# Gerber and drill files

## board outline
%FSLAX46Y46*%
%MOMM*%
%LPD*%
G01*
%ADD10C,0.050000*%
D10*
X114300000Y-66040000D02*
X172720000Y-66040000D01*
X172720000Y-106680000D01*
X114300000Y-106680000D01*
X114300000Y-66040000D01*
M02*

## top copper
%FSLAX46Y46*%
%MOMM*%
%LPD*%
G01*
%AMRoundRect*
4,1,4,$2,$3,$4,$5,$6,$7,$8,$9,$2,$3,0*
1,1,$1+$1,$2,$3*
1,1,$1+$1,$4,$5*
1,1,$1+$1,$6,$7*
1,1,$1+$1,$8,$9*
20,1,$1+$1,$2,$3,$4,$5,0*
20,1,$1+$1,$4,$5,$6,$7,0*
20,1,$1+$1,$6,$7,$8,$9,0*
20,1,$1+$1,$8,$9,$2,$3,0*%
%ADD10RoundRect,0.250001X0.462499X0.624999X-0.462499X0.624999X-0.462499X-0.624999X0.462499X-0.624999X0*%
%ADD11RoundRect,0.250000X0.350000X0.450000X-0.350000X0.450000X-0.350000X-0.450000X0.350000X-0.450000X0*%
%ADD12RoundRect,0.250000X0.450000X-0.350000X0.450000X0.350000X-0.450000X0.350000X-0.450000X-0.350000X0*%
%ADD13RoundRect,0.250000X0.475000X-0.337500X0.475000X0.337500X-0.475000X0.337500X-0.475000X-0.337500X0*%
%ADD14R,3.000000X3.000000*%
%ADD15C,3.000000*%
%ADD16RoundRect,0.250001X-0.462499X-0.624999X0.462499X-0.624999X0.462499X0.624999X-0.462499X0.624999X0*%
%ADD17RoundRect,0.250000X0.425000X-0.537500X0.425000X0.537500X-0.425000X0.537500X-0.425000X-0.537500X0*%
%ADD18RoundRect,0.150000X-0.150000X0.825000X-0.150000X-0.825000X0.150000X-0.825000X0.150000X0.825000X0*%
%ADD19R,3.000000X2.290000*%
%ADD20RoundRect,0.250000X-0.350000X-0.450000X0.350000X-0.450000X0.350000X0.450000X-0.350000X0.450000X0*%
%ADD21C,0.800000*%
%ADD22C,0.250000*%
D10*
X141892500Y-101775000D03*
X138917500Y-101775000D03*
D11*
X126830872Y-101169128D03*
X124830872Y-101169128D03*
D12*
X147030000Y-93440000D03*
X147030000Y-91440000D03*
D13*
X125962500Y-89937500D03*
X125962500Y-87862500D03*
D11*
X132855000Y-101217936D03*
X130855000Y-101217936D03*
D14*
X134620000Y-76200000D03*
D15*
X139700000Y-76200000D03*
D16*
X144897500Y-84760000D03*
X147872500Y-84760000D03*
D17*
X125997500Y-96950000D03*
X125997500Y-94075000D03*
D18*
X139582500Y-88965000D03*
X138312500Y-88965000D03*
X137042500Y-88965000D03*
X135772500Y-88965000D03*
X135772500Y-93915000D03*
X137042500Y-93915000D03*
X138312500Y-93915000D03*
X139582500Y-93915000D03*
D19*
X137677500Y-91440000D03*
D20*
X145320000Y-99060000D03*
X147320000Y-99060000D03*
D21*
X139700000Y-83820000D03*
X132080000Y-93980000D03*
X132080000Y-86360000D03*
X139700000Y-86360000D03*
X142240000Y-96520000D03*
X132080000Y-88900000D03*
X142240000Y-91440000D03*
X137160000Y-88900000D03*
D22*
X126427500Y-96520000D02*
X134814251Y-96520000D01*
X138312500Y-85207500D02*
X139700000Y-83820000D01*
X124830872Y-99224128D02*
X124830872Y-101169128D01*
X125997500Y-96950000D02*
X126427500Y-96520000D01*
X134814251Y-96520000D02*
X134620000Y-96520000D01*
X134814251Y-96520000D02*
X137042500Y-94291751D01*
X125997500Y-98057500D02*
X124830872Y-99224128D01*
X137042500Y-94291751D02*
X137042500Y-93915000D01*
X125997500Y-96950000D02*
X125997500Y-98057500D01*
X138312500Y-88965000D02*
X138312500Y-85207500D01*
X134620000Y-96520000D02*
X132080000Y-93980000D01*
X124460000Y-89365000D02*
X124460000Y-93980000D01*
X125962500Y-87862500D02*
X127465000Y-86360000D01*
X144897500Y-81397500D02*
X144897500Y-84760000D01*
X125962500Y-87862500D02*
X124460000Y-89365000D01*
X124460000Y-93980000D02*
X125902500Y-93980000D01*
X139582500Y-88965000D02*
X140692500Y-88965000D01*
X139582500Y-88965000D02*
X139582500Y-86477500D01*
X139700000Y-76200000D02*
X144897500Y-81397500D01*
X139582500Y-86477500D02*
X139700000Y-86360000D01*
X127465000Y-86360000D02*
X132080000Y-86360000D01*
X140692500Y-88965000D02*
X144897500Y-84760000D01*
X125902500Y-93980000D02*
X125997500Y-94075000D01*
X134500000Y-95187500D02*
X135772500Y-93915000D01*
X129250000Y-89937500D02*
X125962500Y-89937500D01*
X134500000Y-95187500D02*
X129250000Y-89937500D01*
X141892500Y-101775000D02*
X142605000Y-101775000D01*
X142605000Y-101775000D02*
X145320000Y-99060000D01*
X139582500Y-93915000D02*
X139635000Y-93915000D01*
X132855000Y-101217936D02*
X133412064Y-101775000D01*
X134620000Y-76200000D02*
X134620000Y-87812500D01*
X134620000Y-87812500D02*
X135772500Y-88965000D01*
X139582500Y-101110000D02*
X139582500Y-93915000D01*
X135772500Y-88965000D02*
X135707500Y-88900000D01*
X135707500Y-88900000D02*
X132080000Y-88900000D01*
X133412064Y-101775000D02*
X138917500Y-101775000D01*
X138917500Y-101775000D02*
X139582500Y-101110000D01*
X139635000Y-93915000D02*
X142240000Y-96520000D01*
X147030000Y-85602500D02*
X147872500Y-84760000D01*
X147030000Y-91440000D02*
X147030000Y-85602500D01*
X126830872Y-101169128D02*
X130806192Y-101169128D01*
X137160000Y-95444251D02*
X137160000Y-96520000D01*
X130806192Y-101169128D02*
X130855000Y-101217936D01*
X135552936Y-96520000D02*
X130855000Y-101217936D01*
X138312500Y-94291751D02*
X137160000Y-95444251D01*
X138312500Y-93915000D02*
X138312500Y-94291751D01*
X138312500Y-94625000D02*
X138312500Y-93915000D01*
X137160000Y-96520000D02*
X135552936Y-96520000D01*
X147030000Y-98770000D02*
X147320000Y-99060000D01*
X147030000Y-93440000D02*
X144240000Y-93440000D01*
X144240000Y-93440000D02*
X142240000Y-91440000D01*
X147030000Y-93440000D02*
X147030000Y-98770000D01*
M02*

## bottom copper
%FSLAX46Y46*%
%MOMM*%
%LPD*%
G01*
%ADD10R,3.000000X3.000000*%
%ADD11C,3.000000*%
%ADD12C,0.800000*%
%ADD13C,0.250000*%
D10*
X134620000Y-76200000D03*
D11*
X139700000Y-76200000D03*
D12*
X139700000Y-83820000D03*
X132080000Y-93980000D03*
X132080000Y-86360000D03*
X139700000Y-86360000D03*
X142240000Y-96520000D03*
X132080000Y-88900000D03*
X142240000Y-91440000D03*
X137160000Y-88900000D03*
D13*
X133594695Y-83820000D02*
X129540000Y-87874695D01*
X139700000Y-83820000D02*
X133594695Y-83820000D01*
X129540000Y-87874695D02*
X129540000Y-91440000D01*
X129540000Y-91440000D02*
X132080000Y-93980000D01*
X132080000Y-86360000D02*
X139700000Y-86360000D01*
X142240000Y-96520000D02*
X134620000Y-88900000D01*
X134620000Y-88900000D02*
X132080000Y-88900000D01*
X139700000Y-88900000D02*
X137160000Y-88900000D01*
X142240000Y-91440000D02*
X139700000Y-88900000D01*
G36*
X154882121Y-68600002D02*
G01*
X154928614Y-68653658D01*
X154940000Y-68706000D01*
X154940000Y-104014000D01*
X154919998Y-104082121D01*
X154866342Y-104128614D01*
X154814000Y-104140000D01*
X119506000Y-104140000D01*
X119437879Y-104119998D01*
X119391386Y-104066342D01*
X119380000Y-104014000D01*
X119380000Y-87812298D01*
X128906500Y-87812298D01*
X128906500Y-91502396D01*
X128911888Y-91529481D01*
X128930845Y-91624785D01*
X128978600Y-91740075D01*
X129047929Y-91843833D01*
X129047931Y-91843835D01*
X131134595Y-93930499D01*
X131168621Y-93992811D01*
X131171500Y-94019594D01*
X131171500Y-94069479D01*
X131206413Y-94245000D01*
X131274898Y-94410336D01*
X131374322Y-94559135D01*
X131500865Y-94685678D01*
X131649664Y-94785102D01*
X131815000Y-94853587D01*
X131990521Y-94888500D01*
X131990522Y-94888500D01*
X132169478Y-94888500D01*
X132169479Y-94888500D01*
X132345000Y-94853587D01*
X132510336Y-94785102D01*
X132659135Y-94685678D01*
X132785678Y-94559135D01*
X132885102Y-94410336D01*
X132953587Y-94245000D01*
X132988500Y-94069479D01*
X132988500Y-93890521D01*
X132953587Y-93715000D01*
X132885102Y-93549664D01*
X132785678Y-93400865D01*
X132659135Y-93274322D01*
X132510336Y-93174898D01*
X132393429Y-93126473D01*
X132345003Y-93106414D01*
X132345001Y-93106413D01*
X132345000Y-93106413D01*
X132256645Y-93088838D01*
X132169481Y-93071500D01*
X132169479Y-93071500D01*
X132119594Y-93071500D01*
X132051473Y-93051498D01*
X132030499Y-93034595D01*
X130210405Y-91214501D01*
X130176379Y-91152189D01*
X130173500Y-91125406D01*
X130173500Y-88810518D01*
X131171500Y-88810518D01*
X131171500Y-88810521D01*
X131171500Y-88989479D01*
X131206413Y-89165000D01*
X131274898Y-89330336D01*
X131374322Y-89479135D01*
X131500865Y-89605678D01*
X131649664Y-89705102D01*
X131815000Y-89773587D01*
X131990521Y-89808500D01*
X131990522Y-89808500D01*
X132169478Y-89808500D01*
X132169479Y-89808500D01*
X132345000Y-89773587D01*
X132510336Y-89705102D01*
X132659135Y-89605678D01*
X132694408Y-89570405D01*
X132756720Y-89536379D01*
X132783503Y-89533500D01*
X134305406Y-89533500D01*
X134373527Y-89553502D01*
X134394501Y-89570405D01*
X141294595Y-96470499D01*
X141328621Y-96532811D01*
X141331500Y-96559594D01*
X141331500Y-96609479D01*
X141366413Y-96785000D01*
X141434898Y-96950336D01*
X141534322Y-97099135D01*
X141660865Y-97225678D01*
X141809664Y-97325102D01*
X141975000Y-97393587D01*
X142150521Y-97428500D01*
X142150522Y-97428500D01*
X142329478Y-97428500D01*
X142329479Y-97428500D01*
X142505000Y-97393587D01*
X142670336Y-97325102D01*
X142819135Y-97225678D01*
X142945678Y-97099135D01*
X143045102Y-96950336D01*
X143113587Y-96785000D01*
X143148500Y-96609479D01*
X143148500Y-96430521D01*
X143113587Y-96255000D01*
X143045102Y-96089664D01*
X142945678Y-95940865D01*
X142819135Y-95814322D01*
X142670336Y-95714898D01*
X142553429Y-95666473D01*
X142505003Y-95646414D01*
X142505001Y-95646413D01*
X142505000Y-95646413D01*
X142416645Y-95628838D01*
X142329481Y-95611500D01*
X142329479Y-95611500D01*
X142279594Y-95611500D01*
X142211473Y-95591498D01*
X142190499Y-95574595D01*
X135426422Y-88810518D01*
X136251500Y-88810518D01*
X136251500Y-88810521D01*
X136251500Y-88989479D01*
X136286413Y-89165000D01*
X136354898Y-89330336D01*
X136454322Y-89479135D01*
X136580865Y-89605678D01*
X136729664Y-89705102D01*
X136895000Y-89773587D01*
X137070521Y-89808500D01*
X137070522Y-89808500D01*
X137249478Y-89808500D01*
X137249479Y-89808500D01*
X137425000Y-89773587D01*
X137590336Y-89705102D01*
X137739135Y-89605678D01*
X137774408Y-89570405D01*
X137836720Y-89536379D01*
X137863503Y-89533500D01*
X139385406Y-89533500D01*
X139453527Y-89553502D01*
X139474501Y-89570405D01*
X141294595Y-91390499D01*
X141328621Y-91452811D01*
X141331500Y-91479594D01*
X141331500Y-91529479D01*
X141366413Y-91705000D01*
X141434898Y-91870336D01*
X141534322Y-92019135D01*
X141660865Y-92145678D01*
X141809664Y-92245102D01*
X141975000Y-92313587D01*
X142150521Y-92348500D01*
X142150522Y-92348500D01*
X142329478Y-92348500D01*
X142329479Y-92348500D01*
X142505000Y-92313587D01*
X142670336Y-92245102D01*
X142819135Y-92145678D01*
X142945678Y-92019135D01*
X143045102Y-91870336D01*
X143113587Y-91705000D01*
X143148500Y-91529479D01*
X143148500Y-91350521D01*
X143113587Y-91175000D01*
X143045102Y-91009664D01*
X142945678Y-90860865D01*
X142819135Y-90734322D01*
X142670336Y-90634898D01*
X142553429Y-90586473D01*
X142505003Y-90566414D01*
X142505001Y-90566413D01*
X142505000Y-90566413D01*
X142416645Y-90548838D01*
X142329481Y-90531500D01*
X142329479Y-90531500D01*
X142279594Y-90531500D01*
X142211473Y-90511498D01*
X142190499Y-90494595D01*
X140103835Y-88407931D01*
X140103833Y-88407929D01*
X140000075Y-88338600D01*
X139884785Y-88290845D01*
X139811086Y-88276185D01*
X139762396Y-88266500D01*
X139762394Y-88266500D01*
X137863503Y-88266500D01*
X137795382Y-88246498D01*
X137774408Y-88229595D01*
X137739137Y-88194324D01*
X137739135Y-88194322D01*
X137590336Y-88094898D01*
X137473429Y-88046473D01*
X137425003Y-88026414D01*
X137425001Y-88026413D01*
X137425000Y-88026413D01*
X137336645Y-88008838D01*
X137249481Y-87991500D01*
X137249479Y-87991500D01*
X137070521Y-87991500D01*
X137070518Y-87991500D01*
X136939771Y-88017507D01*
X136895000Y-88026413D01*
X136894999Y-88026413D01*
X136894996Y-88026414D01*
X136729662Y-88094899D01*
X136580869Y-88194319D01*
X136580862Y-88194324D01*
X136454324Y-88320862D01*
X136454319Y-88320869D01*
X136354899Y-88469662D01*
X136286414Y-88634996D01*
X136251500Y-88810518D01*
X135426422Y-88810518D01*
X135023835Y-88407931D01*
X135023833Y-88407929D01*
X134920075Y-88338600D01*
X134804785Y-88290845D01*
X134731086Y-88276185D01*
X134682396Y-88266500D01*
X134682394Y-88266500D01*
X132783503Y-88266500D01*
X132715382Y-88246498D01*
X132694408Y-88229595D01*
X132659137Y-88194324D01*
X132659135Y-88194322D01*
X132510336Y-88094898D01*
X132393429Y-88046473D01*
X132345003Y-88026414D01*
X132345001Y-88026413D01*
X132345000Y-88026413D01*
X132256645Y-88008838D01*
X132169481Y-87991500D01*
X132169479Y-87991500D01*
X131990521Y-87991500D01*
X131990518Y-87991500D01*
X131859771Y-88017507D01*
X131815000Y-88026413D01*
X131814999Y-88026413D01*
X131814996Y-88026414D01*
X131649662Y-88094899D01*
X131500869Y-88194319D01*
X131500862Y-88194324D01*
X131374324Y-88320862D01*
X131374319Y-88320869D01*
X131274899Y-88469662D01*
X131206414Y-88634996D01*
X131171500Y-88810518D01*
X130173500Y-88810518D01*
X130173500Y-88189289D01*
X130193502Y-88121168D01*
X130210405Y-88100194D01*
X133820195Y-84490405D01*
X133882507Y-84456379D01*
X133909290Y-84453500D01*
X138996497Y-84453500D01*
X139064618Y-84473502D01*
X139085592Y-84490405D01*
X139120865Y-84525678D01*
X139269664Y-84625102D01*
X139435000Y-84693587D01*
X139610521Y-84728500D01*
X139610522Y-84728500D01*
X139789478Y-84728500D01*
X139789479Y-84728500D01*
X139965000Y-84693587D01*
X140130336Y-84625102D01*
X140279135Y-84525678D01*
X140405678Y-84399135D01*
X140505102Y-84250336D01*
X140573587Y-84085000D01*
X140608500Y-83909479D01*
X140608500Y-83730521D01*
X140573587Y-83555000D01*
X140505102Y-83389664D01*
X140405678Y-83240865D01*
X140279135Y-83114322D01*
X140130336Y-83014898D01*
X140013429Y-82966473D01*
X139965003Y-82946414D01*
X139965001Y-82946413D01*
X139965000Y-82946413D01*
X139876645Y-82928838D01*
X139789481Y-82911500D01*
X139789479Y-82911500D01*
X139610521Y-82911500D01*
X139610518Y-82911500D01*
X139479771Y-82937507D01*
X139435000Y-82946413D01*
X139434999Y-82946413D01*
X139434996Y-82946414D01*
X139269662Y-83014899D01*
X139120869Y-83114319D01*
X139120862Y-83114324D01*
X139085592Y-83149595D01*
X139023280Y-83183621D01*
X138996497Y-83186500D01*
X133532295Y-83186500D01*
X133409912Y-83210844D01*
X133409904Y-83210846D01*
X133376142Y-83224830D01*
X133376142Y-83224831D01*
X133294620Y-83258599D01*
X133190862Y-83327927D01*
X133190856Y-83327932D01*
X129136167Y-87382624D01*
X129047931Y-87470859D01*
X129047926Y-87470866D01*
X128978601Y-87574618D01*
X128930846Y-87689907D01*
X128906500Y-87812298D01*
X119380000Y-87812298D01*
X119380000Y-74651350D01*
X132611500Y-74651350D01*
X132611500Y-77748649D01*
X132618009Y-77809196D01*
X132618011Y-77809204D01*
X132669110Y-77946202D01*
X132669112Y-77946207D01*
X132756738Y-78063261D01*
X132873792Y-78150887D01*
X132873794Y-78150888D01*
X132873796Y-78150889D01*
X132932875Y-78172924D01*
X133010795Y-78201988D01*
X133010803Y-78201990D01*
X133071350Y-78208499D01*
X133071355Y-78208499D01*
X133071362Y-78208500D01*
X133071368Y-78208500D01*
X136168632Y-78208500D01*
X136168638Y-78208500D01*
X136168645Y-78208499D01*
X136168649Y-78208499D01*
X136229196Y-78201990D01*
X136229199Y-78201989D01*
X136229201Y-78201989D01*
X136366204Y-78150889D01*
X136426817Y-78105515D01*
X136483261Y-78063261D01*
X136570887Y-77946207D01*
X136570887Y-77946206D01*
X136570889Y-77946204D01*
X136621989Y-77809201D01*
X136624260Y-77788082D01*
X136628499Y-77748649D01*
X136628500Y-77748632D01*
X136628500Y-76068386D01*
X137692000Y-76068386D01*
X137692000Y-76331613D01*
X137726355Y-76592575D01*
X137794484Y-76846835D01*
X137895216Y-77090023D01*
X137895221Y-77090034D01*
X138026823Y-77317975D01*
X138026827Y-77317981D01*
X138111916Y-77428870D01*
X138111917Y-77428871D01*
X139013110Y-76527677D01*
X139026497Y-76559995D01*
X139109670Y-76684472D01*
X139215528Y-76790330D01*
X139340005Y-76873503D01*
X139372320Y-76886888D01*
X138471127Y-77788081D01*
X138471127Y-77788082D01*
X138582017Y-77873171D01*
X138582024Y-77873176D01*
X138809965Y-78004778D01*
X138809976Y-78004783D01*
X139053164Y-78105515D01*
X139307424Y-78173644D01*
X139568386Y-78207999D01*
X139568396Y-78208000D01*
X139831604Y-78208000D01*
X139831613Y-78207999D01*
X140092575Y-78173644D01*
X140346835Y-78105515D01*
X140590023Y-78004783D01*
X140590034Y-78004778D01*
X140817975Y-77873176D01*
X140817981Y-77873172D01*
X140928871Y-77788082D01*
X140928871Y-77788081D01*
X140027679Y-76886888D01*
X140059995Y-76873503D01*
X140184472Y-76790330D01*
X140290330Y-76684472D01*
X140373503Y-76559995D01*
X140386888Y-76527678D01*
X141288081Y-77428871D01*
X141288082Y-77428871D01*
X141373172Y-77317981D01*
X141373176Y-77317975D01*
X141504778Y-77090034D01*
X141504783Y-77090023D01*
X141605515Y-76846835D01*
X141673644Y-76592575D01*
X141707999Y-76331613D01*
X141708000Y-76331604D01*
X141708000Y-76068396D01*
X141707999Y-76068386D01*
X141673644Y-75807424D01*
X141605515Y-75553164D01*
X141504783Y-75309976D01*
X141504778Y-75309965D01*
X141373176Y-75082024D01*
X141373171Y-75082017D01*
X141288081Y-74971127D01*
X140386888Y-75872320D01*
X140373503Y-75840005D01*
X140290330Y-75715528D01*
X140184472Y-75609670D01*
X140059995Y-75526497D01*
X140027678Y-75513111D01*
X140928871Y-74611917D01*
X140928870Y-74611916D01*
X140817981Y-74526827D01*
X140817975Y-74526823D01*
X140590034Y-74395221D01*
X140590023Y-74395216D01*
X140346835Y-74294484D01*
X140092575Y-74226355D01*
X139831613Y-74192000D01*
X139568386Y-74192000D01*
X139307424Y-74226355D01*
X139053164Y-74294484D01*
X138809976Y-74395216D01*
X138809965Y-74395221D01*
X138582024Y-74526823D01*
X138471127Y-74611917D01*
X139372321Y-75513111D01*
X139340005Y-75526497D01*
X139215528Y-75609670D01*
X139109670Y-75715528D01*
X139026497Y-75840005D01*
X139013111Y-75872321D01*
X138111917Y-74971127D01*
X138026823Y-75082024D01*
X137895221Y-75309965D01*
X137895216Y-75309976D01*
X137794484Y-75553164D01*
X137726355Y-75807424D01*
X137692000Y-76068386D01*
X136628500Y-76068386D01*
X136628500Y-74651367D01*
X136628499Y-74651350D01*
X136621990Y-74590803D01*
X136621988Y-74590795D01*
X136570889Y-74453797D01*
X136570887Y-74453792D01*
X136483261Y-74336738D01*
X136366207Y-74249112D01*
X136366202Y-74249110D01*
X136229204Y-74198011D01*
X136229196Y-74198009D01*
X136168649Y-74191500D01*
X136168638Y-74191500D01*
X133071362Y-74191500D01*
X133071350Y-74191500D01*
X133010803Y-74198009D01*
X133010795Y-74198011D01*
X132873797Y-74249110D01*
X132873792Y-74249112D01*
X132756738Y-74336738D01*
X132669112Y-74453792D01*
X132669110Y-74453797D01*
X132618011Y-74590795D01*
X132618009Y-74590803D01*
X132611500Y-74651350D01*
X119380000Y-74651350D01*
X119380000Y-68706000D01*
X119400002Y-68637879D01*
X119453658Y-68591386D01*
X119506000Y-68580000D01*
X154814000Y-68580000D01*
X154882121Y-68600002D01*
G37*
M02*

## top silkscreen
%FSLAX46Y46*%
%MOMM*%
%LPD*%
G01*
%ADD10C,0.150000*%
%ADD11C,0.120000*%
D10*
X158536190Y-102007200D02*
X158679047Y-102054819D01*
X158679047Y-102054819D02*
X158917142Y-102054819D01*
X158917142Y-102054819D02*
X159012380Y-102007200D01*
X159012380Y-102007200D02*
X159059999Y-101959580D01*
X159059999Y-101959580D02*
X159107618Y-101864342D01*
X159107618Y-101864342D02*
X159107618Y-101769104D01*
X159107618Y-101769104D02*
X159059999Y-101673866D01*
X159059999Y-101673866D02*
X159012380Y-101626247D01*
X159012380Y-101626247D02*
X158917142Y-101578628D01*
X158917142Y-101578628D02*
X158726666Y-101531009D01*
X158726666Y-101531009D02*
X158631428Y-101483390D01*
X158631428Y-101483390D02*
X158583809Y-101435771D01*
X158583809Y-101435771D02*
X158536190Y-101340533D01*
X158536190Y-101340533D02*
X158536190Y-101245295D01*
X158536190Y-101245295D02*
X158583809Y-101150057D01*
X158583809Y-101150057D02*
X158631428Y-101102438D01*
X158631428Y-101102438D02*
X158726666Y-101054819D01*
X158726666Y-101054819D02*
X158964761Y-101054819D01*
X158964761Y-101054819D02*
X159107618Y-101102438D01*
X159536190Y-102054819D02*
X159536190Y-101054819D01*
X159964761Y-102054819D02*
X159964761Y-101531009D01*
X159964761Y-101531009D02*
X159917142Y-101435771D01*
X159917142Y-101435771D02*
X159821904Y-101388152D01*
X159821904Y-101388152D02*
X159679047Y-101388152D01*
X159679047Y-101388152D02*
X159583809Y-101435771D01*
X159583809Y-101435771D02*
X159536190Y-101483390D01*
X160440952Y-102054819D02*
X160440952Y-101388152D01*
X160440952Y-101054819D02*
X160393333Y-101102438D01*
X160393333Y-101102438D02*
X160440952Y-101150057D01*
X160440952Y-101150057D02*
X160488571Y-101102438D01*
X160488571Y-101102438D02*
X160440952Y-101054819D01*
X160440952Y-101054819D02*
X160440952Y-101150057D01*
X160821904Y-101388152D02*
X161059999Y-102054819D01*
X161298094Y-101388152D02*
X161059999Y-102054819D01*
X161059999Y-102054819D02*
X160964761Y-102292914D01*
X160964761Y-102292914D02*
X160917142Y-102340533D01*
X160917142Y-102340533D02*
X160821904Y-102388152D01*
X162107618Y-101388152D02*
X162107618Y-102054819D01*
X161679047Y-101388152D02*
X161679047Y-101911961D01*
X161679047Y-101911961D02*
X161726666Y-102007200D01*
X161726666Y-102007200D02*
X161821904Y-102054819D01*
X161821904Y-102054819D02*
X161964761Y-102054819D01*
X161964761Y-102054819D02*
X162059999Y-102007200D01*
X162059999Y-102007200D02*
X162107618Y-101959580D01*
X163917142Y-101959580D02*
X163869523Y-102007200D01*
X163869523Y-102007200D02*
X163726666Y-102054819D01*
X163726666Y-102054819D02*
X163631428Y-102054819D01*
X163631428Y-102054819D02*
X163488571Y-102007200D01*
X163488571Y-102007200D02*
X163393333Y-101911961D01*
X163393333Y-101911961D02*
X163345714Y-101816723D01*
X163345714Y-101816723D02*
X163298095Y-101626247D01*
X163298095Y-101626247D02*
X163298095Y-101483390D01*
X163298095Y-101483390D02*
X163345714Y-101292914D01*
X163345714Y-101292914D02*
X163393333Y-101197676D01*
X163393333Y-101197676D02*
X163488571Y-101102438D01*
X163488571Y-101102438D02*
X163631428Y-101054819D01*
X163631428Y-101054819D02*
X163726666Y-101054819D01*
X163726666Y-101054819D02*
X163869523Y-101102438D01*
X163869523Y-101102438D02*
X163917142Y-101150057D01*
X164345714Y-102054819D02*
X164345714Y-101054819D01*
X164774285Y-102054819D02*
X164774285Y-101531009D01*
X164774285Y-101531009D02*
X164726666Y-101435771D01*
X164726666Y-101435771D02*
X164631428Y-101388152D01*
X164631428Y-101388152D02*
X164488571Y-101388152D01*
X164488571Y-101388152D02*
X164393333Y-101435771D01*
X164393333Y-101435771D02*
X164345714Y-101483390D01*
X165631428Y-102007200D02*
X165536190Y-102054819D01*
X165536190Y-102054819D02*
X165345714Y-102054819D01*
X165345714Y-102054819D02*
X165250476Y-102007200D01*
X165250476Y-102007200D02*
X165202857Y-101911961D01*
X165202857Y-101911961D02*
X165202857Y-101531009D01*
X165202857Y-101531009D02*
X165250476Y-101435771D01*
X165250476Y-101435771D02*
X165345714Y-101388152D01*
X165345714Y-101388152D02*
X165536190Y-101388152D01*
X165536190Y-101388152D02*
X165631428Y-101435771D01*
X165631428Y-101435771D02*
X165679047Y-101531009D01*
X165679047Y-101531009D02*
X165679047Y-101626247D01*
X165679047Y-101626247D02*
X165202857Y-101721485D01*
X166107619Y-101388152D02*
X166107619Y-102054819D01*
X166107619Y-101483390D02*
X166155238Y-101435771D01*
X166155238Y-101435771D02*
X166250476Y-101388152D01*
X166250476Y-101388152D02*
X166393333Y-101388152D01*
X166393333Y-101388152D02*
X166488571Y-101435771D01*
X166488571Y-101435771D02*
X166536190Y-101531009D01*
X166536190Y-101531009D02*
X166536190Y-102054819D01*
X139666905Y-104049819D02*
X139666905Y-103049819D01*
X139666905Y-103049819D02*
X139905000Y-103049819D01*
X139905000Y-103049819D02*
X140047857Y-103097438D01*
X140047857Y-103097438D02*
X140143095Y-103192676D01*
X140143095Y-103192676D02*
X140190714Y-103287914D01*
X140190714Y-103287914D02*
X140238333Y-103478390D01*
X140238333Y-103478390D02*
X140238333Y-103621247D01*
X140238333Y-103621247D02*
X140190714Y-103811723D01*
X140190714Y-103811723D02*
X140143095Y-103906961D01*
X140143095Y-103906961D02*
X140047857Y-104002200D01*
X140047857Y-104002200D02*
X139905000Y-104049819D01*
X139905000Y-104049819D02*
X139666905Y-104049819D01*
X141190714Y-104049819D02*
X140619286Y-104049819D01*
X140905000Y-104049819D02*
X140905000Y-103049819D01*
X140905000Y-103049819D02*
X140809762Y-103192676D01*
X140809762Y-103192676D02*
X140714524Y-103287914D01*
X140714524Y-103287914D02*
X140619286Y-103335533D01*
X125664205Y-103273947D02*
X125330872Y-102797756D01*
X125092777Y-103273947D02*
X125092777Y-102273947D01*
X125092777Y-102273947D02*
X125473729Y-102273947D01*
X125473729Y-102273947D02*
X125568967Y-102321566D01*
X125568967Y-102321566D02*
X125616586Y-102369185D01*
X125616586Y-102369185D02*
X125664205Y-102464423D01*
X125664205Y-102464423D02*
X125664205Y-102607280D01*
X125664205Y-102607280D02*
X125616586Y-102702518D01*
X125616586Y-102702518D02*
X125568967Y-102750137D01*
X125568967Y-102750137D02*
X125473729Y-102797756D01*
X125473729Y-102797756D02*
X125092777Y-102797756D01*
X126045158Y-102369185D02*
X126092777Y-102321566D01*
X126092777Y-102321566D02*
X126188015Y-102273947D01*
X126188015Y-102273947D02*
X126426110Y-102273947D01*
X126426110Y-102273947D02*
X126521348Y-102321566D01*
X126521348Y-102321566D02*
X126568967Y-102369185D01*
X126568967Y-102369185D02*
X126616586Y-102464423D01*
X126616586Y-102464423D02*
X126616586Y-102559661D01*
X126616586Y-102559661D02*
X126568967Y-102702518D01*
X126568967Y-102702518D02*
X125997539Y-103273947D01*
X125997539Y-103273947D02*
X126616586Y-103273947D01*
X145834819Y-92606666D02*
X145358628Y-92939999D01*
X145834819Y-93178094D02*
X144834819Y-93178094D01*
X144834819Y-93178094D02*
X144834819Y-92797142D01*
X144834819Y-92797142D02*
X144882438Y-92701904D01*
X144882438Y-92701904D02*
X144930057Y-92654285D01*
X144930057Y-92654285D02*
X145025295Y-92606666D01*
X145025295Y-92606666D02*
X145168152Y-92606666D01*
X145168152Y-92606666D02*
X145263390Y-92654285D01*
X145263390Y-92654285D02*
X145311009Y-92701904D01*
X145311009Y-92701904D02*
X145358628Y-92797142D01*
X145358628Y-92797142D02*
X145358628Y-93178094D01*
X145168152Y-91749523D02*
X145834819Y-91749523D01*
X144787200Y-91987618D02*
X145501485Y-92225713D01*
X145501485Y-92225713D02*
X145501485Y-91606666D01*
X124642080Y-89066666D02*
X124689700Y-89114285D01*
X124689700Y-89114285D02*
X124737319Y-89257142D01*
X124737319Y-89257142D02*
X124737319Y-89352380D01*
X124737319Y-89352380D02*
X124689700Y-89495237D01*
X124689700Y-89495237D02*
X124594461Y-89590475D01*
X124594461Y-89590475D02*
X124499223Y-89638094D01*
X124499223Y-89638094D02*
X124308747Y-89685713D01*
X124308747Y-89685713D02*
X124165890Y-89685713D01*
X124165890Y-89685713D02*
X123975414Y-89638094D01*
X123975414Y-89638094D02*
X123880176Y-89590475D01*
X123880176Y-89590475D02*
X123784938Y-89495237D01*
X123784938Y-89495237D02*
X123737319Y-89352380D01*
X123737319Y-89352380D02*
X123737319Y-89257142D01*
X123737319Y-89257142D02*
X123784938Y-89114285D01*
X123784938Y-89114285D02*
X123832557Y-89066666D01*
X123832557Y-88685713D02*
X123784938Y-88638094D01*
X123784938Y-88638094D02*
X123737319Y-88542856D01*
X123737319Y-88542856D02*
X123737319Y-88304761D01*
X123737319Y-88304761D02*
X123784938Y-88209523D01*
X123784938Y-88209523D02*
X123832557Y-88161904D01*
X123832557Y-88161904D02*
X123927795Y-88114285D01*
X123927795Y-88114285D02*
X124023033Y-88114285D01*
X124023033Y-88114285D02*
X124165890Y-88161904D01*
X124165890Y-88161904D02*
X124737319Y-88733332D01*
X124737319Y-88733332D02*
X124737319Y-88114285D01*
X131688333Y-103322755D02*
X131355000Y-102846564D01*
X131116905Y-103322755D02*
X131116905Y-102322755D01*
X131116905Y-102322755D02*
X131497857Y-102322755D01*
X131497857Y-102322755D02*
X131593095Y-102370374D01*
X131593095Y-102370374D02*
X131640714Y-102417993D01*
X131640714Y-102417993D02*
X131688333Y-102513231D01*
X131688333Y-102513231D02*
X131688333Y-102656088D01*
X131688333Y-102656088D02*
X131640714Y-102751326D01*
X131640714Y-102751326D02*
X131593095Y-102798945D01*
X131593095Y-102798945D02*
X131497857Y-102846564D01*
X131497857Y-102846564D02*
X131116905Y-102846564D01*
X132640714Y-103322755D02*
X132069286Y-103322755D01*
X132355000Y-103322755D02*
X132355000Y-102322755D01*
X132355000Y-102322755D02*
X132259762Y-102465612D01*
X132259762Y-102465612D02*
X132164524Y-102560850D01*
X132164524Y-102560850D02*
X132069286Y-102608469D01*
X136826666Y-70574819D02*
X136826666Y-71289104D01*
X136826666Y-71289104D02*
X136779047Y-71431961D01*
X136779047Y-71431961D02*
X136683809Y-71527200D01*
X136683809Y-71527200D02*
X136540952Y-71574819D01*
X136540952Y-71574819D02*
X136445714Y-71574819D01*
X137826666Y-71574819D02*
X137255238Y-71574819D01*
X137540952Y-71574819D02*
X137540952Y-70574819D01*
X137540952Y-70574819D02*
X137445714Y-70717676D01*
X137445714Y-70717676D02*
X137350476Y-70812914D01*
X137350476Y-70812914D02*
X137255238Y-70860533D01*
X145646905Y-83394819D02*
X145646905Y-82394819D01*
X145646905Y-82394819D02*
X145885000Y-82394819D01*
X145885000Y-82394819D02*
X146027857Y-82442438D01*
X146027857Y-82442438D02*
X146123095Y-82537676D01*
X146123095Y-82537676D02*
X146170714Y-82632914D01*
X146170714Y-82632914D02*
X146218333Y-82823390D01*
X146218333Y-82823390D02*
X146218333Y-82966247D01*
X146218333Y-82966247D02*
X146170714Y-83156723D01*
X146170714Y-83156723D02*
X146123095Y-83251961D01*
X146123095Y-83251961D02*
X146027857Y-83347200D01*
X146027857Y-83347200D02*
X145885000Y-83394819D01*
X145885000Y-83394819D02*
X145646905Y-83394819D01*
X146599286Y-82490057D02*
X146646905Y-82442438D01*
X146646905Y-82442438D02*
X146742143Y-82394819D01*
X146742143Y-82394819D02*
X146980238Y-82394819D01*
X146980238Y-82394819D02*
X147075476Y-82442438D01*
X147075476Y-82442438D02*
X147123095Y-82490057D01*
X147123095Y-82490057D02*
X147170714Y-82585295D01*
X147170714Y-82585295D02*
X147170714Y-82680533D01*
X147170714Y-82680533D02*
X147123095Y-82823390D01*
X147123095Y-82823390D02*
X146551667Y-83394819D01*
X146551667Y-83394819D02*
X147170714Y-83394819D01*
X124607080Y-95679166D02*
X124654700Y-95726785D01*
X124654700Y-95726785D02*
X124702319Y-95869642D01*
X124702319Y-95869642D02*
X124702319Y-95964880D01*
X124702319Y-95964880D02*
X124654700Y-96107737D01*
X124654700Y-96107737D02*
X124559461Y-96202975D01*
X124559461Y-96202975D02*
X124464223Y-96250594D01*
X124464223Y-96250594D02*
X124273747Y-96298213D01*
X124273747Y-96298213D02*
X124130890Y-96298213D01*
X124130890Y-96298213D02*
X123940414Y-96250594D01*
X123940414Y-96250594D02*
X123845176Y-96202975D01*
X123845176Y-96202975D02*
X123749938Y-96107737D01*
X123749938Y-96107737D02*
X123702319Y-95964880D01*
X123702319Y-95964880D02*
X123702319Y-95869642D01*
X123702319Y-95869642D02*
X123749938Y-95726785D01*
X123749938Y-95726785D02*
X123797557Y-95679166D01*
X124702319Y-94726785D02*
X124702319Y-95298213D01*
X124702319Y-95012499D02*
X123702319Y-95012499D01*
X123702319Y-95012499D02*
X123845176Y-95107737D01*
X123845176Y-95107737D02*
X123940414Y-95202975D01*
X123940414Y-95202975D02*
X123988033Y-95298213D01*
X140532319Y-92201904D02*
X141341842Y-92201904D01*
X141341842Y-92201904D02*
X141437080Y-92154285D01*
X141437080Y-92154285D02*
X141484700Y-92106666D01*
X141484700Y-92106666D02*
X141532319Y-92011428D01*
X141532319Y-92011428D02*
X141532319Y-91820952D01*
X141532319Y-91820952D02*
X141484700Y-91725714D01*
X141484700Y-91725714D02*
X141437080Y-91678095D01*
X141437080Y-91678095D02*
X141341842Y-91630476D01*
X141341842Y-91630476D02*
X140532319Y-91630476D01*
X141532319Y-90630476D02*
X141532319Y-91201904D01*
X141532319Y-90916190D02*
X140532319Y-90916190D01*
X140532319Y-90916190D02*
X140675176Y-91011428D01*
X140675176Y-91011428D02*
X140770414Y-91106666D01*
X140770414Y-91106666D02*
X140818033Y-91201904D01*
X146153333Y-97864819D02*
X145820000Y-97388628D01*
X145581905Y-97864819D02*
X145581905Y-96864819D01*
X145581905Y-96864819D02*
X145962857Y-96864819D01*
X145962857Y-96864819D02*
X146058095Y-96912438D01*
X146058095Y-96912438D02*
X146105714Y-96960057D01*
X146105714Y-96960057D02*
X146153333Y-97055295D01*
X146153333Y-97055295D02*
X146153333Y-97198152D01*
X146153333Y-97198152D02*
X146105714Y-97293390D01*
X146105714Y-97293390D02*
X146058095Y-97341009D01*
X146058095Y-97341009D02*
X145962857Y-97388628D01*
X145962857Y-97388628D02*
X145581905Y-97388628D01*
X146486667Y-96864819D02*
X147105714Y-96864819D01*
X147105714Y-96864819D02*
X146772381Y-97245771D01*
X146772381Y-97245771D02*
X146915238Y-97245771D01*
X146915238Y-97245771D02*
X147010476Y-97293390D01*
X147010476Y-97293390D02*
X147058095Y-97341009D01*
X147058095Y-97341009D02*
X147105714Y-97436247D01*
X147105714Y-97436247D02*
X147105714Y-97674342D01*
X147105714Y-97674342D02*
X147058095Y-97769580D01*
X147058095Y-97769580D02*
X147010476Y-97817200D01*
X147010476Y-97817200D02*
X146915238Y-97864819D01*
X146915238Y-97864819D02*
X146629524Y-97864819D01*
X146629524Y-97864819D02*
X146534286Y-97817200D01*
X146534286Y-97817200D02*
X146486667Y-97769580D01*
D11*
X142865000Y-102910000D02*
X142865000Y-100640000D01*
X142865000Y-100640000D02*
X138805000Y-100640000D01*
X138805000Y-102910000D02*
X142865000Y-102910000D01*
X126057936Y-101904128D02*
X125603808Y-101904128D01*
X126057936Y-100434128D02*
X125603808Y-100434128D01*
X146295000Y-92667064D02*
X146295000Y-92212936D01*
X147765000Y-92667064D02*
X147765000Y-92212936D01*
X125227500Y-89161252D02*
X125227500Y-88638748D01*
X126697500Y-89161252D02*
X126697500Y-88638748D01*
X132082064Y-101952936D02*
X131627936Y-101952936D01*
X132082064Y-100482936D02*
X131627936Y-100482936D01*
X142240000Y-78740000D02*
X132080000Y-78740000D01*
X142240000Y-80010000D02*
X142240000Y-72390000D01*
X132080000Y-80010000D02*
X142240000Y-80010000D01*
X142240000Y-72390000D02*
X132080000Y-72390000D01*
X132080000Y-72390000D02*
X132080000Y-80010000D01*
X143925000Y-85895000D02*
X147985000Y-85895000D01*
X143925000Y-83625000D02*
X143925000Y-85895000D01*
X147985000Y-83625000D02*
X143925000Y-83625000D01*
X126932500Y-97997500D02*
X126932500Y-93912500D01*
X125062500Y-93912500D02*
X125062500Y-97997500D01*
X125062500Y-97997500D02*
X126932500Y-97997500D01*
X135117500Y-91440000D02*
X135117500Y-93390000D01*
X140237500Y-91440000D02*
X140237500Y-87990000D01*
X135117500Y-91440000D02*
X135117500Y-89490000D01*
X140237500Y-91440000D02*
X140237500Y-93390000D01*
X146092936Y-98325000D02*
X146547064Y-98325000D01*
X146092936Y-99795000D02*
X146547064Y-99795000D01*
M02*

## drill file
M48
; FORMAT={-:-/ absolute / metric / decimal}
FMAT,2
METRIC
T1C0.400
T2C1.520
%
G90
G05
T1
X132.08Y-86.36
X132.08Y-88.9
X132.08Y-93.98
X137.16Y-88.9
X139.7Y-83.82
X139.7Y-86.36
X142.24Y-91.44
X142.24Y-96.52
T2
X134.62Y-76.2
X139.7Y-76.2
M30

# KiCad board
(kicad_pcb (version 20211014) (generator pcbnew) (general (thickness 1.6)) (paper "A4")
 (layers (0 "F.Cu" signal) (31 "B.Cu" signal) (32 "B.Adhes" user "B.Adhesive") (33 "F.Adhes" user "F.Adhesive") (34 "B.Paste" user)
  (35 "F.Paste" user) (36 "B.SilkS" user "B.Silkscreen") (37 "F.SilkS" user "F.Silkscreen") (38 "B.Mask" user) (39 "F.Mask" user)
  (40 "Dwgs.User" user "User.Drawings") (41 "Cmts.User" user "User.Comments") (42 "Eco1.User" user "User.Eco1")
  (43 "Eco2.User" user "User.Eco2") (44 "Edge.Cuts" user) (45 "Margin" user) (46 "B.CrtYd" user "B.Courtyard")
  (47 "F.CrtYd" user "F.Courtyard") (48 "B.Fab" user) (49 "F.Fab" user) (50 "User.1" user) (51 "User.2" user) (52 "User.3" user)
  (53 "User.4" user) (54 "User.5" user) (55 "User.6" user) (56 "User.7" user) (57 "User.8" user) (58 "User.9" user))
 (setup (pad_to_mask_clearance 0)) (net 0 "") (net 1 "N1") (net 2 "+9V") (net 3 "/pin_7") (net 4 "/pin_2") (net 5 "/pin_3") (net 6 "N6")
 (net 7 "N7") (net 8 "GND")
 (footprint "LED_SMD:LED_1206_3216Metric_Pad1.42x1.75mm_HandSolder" (layer "F.Cu") (at 140.405 101.775 180)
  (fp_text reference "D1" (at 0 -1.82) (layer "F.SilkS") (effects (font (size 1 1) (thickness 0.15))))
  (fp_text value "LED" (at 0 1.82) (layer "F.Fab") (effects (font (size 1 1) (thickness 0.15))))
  (fp_line (start -2.46 -1.135) (end -2.46 1.135) (layer "F.SilkS") (width 0.12))
  (fp_line (start -2.46 1.135) (end 1.6 1.135) (layer "F.SilkS") (width 0.12))
  (fp_line (start 1.6 -1.135) (end -2.46 -1.135) (layer "F.SilkS") (width 0.12))
  (pad "1" smd roundrect (at -1.4875 0 180) (size 1.425 1.75) (layers "F.Cu" "F.Paste" "F.Mask") (roundrect_rratio 0.1754392982)
   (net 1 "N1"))
  (pad "2" smd roundrect (at 1.4875 0 180) (size 1.425 1.75) (layers "F.Cu" "F.Paste" "F.Mask") (roundrect_rratio 0.1754392982)
   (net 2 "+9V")))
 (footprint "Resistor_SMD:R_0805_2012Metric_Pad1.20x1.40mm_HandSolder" (layer "F.Cu") (at 125.830872 101.169128 180)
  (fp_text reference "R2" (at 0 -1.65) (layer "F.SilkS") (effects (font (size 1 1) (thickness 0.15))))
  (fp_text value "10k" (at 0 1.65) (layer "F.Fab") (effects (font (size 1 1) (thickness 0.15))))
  (fp_line (start -0.227064 -0.735) (end 0.227064 -0.735) (layer "F.SilkS") (width 0.12))
  (fp_line (start -0.227064 0.735) (end 0.227064 0.735) (layer "F.SilkS") (width 0.12))
  (pad "1" smd roundrect (at -1 0 180) (size 1.2 1.4) (layers "F.Cu" "F.Paste" "F.Mask") (roundrect_rratio 0.2083333333) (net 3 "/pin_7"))
  (pad "2" smd roundrect (at 1 0 180) (size 1.2 1.4) (layers "F.Cu" "F.Paste" "F.Mask") (roundrect_rratio 0.2083333333) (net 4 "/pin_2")))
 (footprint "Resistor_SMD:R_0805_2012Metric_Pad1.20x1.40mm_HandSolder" (layer "F.Cu") (at 147.03 92.44 90)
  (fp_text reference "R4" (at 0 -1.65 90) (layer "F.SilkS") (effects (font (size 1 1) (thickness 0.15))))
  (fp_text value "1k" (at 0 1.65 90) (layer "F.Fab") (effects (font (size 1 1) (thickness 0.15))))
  (fp_line (start -0.227064 -0.735) (end 0.227064 -0.735) (layer "F.SilkS") (width 0.12))
  (fp_line (start -0.227064 0.735) (end 0.227064 0.735) (layer "F.SilkS") (width 0.12))
  (pad "1" smd roundrect (at -1 0 90) (size 1.2 1.4) (layers "F.Cu" "F.Paste" "F.Mask") (roundrect_rratio 0.2083333333) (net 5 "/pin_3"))
  (pad "2" smd roundrect (at 1 0 90) (size 1.2 1.4) (layers "F.Cu" "F.Paste" "F.Mask") (roundrect_rratio 0.2083333333) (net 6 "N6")))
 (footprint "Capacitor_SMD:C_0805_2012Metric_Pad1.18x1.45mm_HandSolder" (layer "F.Cu") (at 125.9625 88.9 90)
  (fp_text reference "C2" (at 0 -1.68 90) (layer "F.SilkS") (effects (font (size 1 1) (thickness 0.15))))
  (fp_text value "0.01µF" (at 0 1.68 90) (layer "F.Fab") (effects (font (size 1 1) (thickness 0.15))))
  (fp_line (start -0.261252 -0.735) (end 0.261252 -0.735) (layer "F.SilkS") (width 0.12))
  (fp_line (start -0.261252 0.735) (end 0.261252 0.735) (layer "F.SilkS") (width 0.12))
  (pad "1" smd roundrect (at -1.0375 0 90) (size 1.175 1.45) (layers "F.Cu" "F.Paste" "F.Mask") (roundrect_rratio 0.2127659574) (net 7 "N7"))
  (pad "2" smd roundrect (at 1.0375 0 90) (size 1.175 1.45) (layers "F.Cu" "F.Paste" "F.Mask") (roundrect_rratio 0.2127659574) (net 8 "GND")))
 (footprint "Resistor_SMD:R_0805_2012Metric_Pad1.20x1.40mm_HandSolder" (layer "F.Cu") (at 131.855 101.217936 180)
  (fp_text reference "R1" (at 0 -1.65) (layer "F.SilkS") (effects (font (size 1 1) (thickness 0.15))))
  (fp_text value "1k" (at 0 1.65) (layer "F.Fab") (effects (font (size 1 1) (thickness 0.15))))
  (fp_line (start -0.227064 -0.735) (end 0.227064 -0.735) (layer "F.SilkS") (width 0.12))
  (fp_line (start -0.227064 0.735) (end 0.227064 0.735) (layer "F.SilkS") (width 0.12))
  (pad "1" smd roundrect (at -1 0 180) (size 1.2 1.4) (layers "F.Cu" "F.Paste" "F.Mask") (roundrect_rratio 0.2083333333) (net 2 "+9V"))
  (pad "2" smd roundrect (at 1 0 180) (size 1.2 1.4) (layers "F.Cu" "F.Paste" "F.Mask") (roundrect_rratio 0.2083333333) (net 3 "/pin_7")))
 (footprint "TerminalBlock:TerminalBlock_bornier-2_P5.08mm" (layer "F.Cu") (at 134.62 76.2)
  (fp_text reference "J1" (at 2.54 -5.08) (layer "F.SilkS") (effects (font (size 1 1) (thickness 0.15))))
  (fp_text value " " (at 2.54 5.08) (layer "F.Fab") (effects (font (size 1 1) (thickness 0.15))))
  (fp_line (start 7.62 2.54) (end -2.54 2.54) (layer "F.SilkS") (width 0.12))
  (fp_line (start 7.62 3.81) (end 7.62 -3.81) (layer "F.SilkS") (width 0.12))
  (fp_line (start -2.54 3.81) (end 7.62 3.81) (layer "F.SilkS") (width 0.12))
  (fp_line (start 7.62 -3.81) (end -2.54 -3.81) (layer "F.SilkS") (width 0.12))
  (fp_line (start -2.54 -3.81) (end -2.54 3.81) (layer "F.SilkS") (width 0.12))
  (pad "1" thru_hole rect (at 0 0) (size 3 3) (drill 1.52) (layers *.Cu *.Mask) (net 2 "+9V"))
  (pad "2" thru_hole circle (at 5.08 0) (size 3 3) (drill 1.52) (layers *.Cu *.Mask) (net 8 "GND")))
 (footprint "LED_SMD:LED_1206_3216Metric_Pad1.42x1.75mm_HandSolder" (layer "F.Cu") (at 146.385 84.76)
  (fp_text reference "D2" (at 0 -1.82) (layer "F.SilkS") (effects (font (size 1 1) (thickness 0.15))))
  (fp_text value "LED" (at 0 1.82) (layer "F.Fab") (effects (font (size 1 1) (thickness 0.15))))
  (fp_line (start -2.46 1.135) (end 1.6 1.135) (layer "F.SilkS") (width 0.12))
  (fp_line (start -2.46 -1.135) (end -2.46 1.135) (layer "F.SilkS") (width 0.12))
  (fp_line (start 1.6 -1.135) (end -2.46 -1.135) (layer "F.SilkS") (width 0.12))
  (pad "1" smd roundrect (at -1.4875 0) (size 1.425 1.75) (layers "F.Cu" "F.Paste" "F.Mask") (roundrect_rratio 0.1754392982) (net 8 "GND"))
  (pad "2" smd roundrect (at 1.4875 0) (size 1.425 1.75) (layers "F.Cu" "F.Paste" "F.Mask") (roundrect_rratio 0.1754392982) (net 6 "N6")))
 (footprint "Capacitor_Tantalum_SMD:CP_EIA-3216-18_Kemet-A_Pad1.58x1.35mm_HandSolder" (layer "F.Cu") (at 125.9975 95.5125 90)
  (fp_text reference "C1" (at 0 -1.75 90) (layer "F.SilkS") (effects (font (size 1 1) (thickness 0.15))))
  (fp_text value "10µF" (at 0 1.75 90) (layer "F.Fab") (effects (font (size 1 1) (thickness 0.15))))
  (fp_line (start -2.485 0.935) (end 1.6 0.935) (layer "F.SilkS") (width 0.12))
  (fp_line (start 1.6 -0.935) (end -2.485 -0.935) (layer "F.SilkS") (width 0.12))
  (fp_line (start -2.485 -0.935) (end -2.485 0.935) (layer "F.SilkS") (width 0.12))
  (pad "1" smd roundrect (at -1.4375 0 90) (size 1.575 1.35) (layers "F.Cu" "F.Paste" "F.Mask") (roundrect_rratio 0.1851851852)
   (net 4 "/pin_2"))
  (pad "2" smd roundrect (at 1.4375 0 90) (size 1.575 1.35) (layers "F.Cu" "F.Paste" "F.Mask") (roundrect_rratio 0.1851851852) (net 8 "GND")))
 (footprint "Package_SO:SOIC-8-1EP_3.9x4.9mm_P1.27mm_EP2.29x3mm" (layer "F.Cu") (at 137.6775 91.44 -90)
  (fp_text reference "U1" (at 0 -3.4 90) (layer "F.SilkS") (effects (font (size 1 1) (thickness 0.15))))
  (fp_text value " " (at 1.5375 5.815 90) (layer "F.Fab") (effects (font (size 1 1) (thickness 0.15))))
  (fp_line (start 0 2.56) (end 1.95 2.56) (layer "F.SilkS") (width 0.12))
  (fp_line (start 0 -2.56) (end -3.45 -2.56) (layer "F.SilkS") (width 0.12))
  (fp_line (start 0 2.56) (end -1.95 2.56) (layer "F.SilkS") (width 0.12))
  (fp_line (start 0 -2.56) (end 1.95 -2.56) (layer "F.SilkS") (width 0.12))
  (pad "" smd roundrect (at -0.57 -0.75 270) (size 0.92 1.21) (layers "F.Paste") (roundrect_rratio 0.25))
  (pad "" smd roundrect (at 0.57 -0.75 270) (size 0.92 1.21) (layers "F.Paste") (roundrect_rratio 0.25))
  (pad "" smd roundrect (at -0.57 0.75 270) (size 0.92 1.21) (layers "F.Paste") (roundrect_rratio 0.25))
  (pad "" smd roundrect (at 0.57 0.75 270) (size 0.92 1.21) (layers "F.Paste") (roundrect_rratio 0.25))
  (pad "1" smd roundrect (at -2.475 -1.905 270) (size 1.95 0.6) (layers "F.Cu" "F.Paste" "F.Mask") (roundrect_rratio 0.25) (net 8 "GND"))
  (pad "2" smd roundrect (at -2.475 -0.635 270) (size 1.95 0.6) (layers "F.Cu" "F.Paste" "F.Mask") (roundrect_rratio 0.25) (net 4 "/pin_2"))
  (pad "3" smd roundrect (at -2.475 0.635 270) (size 1.95 0.6) (layers "F.Cu" "F.Paste" "F.Mask") (roundrect_rratio 0.25) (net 5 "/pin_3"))
  (pad "4" smd roundrect (at -2.475 1.905 270) (size 1.95 0.6) (layers "F.Cu" "F.Paste" "F.Mask") (roundrect_rratio 0.25) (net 2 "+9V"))
  (pad "5" smd roundrect (at 2.475 1.905 270) (size 1.95 0.6) (layers "F.Cu" "F.Paste" "F.Mask") (roundrect_rratio 0.25) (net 7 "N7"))
  (pad "6" smd roundrect (at 2.475 0.635 270) (size 1.95 0.6) (layers "F.Cu" "F.Paste" "F.Mask") (roundrect_rratio 0.25) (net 4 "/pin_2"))
  (pad "7" smd roundrect (at 2.475 -0.635 270) (size 1.95 0.6) (layers "F.Cu" "F.Paste" "F.Mask") (roundrect_rratio 0.25) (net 3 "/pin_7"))
  (pad "8" smd roundrect (at 2.475 -1.905 270) (size 1.95 0.6) (layers "F.Cu" "F.Paste" "F.Mask") (roundrect_rratio 0.25) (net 2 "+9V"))
  (pad "9" smd rect (at 0 0 270) (size 2.29 3) (layers "F.Cu" "F.Mask")))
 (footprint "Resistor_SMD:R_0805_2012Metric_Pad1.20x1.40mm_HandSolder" (layer "F.Cu") (at 146.32 99.06)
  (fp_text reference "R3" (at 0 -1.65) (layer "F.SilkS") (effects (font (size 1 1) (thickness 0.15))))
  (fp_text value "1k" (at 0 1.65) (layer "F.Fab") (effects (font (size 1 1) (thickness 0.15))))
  (fp_line (start -0.227064 -0.735) (end 0.227064 -0.735) (layer "F.SilkS") (width 0.12))
  (fp_line (start -0.227064 0.735) (end 0.227064 0.735) (layer "F.SilkS") (width 0.12))
  (pad "1" smd roundrect (at -1 0) (size 1.2 1.4) (layers "F.Cu" "F.Paste" "F.Mask") (roundrect_rratio 0.2083333333) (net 1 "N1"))
  (pad "2" smd roundrect (at 1 0) (size 1.2 1.4) (layers "F.Cu" "F.Paste" "F.Mask") (roundrect_rratio 0.2083333333) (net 5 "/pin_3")))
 (gr_rect (start 114.3 66.04) (end 172.72 106.68) (layer "Edge.Cuts") (width 0.05) (fill none))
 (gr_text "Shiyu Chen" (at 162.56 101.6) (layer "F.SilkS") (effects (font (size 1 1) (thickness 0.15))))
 (segment (start 126.4275 96.52) (end 134.814251 96.52) (width 0.25) (layer "F.Cu") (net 4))
 (segment (start 138.3125 85.2075) (end 139.7 83.82) (width 0.25) (layer "F.Cu") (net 4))
 (segment (start 124.830872 99.224128) (end 124.830872 101.169128) (width 0.25) (layer "F.Cu") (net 4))
 (segment (start 125.9975 96.95) (end 126.4275 96.52) (width 0.25) (layer "F.Cu") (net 4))
 (segment (start 134.814251 96.52) (end 134.62 96.52) (width 0.25) (layer "F.Cu") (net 4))
 (segment (start 134.814251 96.52) (end 137.0425 94.291751) (width 0.25) (layer "F.Cu") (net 4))
 (segment (start 125.9975 98.0575) (end 124.830872 99.224128) (width 0.25) (layer "F.Cu") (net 4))
 (segment (start 137.0425 94.291751) (end 137.0425 93.915) (width 0.25) (layer "F.Cu") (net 4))
 (segment (start 125.9975 96.95) (end 125.9975 98.0575) (width 0.25) (layer "F.Cu") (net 4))
 (segment (start 138.3125 88.965) (end 138.3125 85.2075) (width 0.25) (layer "F.Cu") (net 4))
 (segment (start 134.62 96.52) (end 132.08 93.98) (width 0.25) (layer "F.Cu") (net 4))
 (via (at 139.7 83.82) (size 0.8) (drill 0.4) (layers "F.Cu" "B.Cu") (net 4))
 (via (at 132.08 93.98) (size 0.8) (drill 0.4) (layers "F.Cu" "B.Cu") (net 4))
 (segment (start 133.594695 83.82) (end 129.54 87.874695) (width 0.25) (layer "B.Cu") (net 4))
 (segment (start 139.7 83.82) (end 133.594695 83.82) (width 0.25) (layer "B.Cu") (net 4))
 (segment (start 129.54 87.874695) (end 129.54 91.44) (width 0.25) (layer "B.Cu") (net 4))
 (segment (start 129.54 91.44) (end 132.08 93.98) (width 0.25) (layer "B.Cu") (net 4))
 (segment (start 124.46 89.365) (end 124.46 93.98) (width 0.25) (layer "F.Cu") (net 8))
 (segment (start 125.9625 87.8625) (end 127.465 86.36) (width 0.25) (layer "F.Cu") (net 8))
 (segment (start 144.8975 81.3975) (end 144.8975 84.76) (width 0.25) (layer "F.Cu") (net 8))
 (segment (start 125.9625 87.8625) (end 124.46 89.365) (width 0.25) (layer "F.Cu") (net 8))
 (segment (start 124.46 93.98) (end 125.9025 93.98) (width 0.25) (layer "F.Cu") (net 8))
 (segment (start 139.5825 88.965) (end 140.6925 88.965) (width 0.25) (layer "F.Cu") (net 8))
 (segment (start 139.5825 88.965) (end 139.5825 86.4775) (width 0.25) (layer "F.Cu") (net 8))
 (segment (start 139.7 76.2) (end 144.8975 81.3975) (width 0.25) (layer "F.Cu") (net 8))
 (segment (start 139.5825 86.4775) (end 139.7 86.36) (width 0.25) (layer "F.Cu") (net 8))
 (segment (start 127.465 86.36) (end 132.08 86.36) (width 0.25) (layer "F.Cu") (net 8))
 (segment (start 140.6925 88.965) (end 144.8975 84.76) (width 0.25) (layer "F.Cu") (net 8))
 (segment (start 125.9025 93.98) (end 125.9975 94.075) (width 0.25) (layer "F.Cu") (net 8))
 (via (at 132.08 86.36) (size 0.8) (drill 0.4) (layers "F.Cu" "B.Cu") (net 8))
 (via (at 139.7 86.36) (size 0.8) (drill 0.4) (layers "F.Cu" "B.Cu") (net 8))
 (segment (start 132.08 86.36) (end 139.7 86.36) (width 0.25) (layer "B.Cu") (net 8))
 (segment (start 134.5 95.1875) (end 135.7725 93.915) (width 0.25) (layer "F.Cu") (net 7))
 (segment (start 129.25 89.9375) (end 125.9625 89.9375) (width 0.25) (layer "F.Cu") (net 7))
 (segment (start 134.5 95.1875) (end 129.25 89.9375) (width 0.25) (layer "F.Cu") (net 7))
 (segment (start 141.8925 101.775) (end 142.605 101.775) (width 0.25) (layer "F.Cu") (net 1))
 (segment (start 142.605 101.775) (end 145.32 99.06) (width 0.25) (layer "F.Cu") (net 1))
 (segment (start 139.5825 93.915) (end 139.635 93.915) (width 0.25) (layer "F.Cu") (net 2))
 (segment (start 132.855 101.217936) (end 133.412064 101.775) (width 0.25) (layer "F.Cu") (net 2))
 (segment (start 134.62 76.2) (end 134.62 87.8125) (width 0.25) (layer "F.Cu") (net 2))
 (segment (start 134.62 87.8125) (end 135.7725 88.965) (width 0.25) (layer "F.Cu") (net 2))
 (segment (start 139.5825 101.11) (end 139.5825 93.915) (width 0.25) (layer "F.Cu") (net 2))
 (segment (start 135.7725 88.965) (end 135.7075 88.9) (width 0.25) (layer "F.Cu") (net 2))
 (segment (start 135.7075 88.9) (end 132.08 88.9) (width 0.25) (layer "F.Cu") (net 2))
 (segment (start 133.412064 101.775) (end 138.9175 101.775) (width 0.25) (layer "F.Cu") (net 2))
 (segment (start 138.9175 101.775) (end 139.5825 101.11) (width 0.25) (layer "F.Cu") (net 2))
 (segment (start 139.635 93.915) (end 142.24 96.52) (width 0.25) (layer "F.Cu") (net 2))
 (via (at 142.24 96.52) (size 0.8) (drill 0.4) (layers "F.Cu" "B.Cu") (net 2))
 (via (at 132.08 88.9) (size 0.8) (drill 0.4) (layers "F.Cu" "B.Cu") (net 2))
 (segment (start 142.24 96.52) (end 134.62 88.9) (width 0.25) (layer "B.Cu") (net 2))
 (segment (start 134.62 88.9) (end 132.08 88.9) (width 0.25) (layer "B.Cu") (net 2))
 (segment (start 147.03 85.6025) (end 147.8725 84.76) (width 0.25) (layer "F.Cu") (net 6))
 (segment (start 147.03 91.44) (end 147.03 85.6025) (width 0.25) (layer "F.Cu") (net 6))
 (segment (start 126.830872 101.169128) (end 130.806192 101.169128) (width 0.25) (layer "F.Cu") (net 3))
 (segment (start 137.16 95.444251) (end 137.16 96.52) (width 0.25) (layer "F.Cu") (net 3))
 (segment (start 130.806192 101.169128) (end 130.855 101.217936) (width 0.25) (layer "F.Cu") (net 3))
 (segment (start 135.552936 96.52) (end 130.855 101.217936) (width 0.25) (layer "F.Cu") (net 3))
 (segment (start 138.3125 94.291751) (end 137.16 95.444251) (width 0.25) (layer "F.Cu") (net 3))
 (segment (start 138.3125 93.915) (end 138.3125 94.291751) (width 0.25) (layer "F.Cu") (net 3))
 (segment (start 138.3125 94.625) (end 138.3125 93.915) (width 0.25) (layer "F.Cu") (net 3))
 (segment (start 137.16 96.52) (end 135.552936 96.52) (width 0.25) (layer "F.Cu") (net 3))
 (segment (start 147.03 98.77) (end 147.32 99.06) (width 0.25) (layer "F.Cu") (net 5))
 (segment (start 147.03 93.44) (end 144.24 93.44) (width 0.25) (layer "F.Cu") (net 5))
 (segment (start 144.24 93.44) (end 142.24 91.44) (width 0.25) (layer "F.Cu") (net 5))
 (segment (start 147.03 93.44) (end 147.03 98.77) (width 0.25) (layer "F.Cu") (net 5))
 (via (at 142.24 91.44) (size 0.8) (drill 0.4) (layers "F.Cu" "B.Cu") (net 5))
 (via (at 137.16 88.9) (size 0.8) (drill 0.4) (layers "F.Cu" "B.Cu") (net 5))
 (segment (start 139.7 88.9) (end 137.16 88.9) (width 0.25) (layer "B.Cu") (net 5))
 (segment (start 142.24 91.44) (end 139.7 88.9) (width 0.25) (layer "B.Cu") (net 5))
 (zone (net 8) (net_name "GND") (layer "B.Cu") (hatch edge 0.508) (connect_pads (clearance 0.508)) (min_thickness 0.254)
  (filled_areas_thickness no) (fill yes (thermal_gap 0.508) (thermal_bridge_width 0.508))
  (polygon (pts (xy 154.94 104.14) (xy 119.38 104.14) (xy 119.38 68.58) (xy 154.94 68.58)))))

